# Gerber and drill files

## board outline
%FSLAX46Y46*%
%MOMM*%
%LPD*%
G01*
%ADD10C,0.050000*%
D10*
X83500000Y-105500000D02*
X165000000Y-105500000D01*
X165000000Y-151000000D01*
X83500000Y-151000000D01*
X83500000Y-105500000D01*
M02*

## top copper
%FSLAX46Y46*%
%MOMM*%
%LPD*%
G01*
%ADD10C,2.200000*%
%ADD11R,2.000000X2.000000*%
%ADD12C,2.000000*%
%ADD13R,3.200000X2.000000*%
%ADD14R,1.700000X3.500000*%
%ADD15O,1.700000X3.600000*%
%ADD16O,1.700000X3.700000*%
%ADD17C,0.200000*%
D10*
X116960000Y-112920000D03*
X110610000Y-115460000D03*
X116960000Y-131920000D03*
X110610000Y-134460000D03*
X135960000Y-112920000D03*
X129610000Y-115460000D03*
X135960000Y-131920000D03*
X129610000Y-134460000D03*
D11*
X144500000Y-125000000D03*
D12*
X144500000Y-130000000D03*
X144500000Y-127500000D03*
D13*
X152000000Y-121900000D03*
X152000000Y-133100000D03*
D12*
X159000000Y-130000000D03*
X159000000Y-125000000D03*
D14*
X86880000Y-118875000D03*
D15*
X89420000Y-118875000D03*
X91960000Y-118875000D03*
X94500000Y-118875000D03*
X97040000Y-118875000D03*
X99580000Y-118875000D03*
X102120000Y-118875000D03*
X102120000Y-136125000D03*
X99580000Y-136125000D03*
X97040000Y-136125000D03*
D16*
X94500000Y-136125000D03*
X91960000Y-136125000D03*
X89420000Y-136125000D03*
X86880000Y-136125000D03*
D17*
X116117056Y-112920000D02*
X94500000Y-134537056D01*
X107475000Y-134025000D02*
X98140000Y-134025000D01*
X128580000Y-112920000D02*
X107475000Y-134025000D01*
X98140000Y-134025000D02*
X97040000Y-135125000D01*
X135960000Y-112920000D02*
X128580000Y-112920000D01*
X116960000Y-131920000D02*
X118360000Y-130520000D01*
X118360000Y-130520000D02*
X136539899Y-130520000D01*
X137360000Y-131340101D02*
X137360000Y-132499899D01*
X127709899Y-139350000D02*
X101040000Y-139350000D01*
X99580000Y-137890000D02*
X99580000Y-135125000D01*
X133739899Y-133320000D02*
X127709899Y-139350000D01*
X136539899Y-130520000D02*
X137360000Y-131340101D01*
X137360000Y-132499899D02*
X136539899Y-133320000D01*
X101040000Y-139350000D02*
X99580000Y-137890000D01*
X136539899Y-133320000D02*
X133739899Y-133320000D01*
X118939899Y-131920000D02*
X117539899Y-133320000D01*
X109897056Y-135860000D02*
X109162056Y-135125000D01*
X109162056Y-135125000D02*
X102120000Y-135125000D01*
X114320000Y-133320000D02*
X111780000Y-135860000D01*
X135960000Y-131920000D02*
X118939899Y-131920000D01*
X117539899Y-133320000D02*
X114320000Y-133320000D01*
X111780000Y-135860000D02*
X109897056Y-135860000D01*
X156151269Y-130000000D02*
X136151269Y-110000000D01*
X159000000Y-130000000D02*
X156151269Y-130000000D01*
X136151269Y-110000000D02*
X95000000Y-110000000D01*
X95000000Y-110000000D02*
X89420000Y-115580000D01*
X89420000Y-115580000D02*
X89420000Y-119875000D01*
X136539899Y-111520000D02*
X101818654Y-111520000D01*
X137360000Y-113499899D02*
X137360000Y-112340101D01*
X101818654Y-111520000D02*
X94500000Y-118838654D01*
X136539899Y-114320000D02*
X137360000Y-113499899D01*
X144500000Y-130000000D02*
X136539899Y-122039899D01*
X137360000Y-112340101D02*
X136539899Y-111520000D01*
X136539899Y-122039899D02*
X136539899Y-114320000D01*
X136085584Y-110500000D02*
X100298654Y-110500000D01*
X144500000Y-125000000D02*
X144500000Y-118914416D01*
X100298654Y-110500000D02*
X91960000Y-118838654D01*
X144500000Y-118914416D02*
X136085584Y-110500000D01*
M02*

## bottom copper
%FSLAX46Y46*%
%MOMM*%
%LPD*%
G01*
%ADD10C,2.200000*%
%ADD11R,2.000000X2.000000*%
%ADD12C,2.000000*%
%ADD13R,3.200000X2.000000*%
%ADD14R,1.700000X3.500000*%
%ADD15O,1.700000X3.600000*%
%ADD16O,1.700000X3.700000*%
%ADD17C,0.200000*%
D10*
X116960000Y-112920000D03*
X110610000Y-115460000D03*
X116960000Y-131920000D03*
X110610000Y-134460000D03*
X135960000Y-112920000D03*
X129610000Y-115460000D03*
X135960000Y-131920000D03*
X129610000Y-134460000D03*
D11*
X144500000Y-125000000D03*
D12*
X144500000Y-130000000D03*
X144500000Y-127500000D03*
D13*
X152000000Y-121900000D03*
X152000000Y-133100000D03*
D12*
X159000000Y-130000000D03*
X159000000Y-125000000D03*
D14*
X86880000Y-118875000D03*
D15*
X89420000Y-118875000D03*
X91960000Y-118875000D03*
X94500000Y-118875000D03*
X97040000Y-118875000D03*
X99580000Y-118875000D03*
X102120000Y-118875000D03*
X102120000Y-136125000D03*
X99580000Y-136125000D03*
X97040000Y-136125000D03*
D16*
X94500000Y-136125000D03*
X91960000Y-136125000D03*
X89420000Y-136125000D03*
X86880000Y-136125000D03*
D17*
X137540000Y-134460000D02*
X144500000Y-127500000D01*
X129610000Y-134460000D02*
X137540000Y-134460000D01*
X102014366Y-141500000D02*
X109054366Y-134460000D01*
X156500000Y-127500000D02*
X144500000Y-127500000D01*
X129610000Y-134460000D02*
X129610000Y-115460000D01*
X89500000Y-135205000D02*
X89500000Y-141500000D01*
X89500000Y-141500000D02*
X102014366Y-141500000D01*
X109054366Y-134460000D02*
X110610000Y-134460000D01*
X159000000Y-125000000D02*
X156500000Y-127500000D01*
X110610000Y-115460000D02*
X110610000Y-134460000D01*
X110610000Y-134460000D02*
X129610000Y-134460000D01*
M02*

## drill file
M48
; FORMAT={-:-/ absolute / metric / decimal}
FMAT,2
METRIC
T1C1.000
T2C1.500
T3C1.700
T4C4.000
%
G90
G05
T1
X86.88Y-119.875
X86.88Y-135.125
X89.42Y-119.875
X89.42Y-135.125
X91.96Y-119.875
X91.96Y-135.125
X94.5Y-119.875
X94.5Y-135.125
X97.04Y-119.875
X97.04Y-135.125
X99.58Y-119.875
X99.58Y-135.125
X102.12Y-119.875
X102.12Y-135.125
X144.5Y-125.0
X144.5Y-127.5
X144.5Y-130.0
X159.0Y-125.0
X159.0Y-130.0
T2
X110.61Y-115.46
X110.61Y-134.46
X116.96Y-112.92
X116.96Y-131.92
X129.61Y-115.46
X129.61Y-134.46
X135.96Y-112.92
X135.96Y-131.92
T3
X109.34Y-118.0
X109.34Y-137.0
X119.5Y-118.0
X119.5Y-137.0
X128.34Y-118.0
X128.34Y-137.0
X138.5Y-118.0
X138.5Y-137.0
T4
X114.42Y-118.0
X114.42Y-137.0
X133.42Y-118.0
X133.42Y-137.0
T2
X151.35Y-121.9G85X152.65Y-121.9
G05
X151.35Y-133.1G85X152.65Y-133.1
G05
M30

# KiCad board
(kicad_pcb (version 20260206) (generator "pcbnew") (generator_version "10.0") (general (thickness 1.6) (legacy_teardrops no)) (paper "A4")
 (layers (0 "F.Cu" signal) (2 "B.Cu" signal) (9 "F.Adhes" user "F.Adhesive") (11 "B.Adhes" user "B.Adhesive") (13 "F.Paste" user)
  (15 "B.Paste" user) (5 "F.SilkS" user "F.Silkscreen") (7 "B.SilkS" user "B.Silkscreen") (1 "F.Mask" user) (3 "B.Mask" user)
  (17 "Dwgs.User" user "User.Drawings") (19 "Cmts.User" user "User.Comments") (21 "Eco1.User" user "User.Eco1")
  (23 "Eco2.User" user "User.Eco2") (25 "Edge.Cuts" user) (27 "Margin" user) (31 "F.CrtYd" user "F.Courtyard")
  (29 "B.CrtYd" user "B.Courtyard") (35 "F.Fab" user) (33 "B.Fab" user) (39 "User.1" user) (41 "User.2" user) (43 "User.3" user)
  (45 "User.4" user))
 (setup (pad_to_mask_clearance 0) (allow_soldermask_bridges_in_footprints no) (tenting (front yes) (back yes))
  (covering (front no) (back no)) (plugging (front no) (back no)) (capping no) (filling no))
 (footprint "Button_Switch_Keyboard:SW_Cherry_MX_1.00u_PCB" (layer "F.Cu") (at 116.96 112.92)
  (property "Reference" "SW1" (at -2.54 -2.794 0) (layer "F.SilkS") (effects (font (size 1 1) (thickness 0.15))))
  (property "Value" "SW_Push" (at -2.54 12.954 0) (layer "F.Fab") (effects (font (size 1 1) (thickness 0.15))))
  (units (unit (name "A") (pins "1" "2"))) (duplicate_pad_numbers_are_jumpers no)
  (pad "" np_thru_hole circle (at -7.62 5.08) (size 1.7 1.7) (drill 1.7) (layers "*.Cu" "*.Mask"))
  (pad "" np_thru_hole circle (at -2.54 5.08) (size 4 4) (drill 4) (layers "*.Cu" "*.Mask"))
  (pad "" np_thru_hole circle (at 2.54 5.08) (size 1.7 1.7) (drill 1.7) (layers "*.Cu" "*.Mask"))
  (pad "1" thru_hole circle (at 0 0) (size 2.2 2.2) (drill 1.5) (layers "*.Cu" "*.Mask") (remove_unused_layers no)
   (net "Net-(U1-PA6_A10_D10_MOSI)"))
  (pad "2" thru_hole circle (at -6.35 2.54) (size 2.2 2.2) (drill 1.5) (layers "*.Cu" "*.Mask") (remove_unused_layers no)
   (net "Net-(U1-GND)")))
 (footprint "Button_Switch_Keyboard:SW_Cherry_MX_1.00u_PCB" (layer "F.Cu") (at 116.96 131.92)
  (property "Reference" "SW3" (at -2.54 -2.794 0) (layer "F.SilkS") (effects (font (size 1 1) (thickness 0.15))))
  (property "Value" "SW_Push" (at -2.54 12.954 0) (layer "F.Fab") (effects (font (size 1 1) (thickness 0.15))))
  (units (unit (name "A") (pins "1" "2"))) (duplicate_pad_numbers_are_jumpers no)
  (pad "" np_thru_hole circle (at -7.62 5.08) (size 1.7 1.7) (drill 1.7) (layers "*.Cu" "*.Mask"))
  (pad "" np_thru_hole circle (at -2.54 5.08) (size 4 4) (drill 4) (layers "*.Cu" "*.Mask"))
  (pad "" np_thru_hole circle (at 2.54 5.08) (size 1.7 1.7) (drill 1.7) (layers "*.Cu" "*.Mask"))
  (pad "1" thru_hole circle (at 0 0) (size 2.2 2.2) (drill 1.5) (layers "*.Cu" "*.Mask") (remove_unused_layers no)
   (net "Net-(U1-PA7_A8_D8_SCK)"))
  (pad "2" thru_hole circle (at -6.35 2.54) (size 2.2 2.2) (drill 1.5) (layers "*.Cu" "*.Mask") (remove_unused_layers no)
   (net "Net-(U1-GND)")))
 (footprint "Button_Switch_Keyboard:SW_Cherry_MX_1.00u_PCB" (layer "F.Cu") (at 135.96 112.92)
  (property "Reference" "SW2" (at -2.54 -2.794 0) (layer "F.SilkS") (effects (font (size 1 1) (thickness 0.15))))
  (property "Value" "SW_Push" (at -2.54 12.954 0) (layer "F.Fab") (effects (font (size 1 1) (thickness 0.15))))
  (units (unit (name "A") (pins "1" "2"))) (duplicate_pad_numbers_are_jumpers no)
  (pad "" np_thru_hole circle (at -7.62 5.08) (size 1.7 1.7) (drill 1.7) (layers "*.Cu" "*.Mask"))
  (pad "" np_thru_hole circle (at -2.54 5.08) (size 4 4) (drill 4) (layers "*.Cu" "*.Mask"))
  (pad "" np_thru_hole circle (at 2.54 5.08) (size 1.7 1.7) (drill 1.7) (layers "*.Cu" "*.Mask"))
  (pad "1" thru_hole circle (at 0 0) (size 2.2 2.2) (drill 1.5) (layers "*.Cu" "*.Mask") (remove_unused_layers no)
   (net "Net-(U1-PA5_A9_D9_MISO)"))
  (pad "2" thru_hole circle (at -6.35 2.54) (size 2.2 2.2) (drill 1.5) (layers "*.Cu" "*.Mask") (remove_unused_layers no)
   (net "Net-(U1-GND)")))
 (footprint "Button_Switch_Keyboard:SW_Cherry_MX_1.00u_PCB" (layer "F.Cu") (at 135.96 131.92)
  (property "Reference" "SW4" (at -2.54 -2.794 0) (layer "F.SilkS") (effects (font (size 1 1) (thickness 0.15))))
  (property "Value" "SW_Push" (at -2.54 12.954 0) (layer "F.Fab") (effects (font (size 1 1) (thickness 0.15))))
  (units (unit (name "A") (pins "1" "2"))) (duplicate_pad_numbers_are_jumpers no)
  (pad "" np_thru_hole circle (at -7.62 5.08) (size 1.7 1.7) (drill 1.7) (layers "*.Cu" "*.Mask"))
  (pad "" np_thru_hole circle (at -2.54 5.08) (size 4 4) (drill 4) (layers "*.Cu" "*.Mask"))
  (pad "" np_thru_hole circle (at 2.54 5.08) (size 1.7 1.7) (drill 1.7) (layers "*.Cu" "*.Mask"))
  (pad "1" thru_hole circle (at 0 0) (size 2.2 2.2) (drill 1.5) (layers "*.Cu" "*.Mask") (remove_unused_layers no)
   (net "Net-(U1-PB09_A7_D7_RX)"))
  (pad "2" thru_hole circle (at -6.35 2.54) (size 2.2 2.2) (drill 1.5) (layers "*.Cu" "*.Mask") (remove_unused_layers no)
   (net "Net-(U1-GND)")))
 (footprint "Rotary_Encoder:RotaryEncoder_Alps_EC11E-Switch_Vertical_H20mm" (layer "F.Cu") (at 144.5 125)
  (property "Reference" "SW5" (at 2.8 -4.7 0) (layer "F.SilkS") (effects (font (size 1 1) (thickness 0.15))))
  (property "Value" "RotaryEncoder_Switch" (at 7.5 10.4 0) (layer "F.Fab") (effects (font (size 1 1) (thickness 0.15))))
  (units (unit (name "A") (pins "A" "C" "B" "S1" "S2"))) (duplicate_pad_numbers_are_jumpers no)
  (pad "A" thru_hole rect (at 0 0) (size 2 2) (drill 1) (layers "*.Cu" "*.Mask") (remove_unused_layers no) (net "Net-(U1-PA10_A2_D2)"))
  (pad "B" thru_hole circle (at 0 5) (size 2 2) (drill 1) (layers "*.Cu" "*.Mask") (remove_unused_layers no) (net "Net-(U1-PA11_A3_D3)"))
  (pad "C" thru_hole circle (at 0 2.5) (size 2 2) (drill 1) (layers "*.Cu" "*.Mask") (remove_unused_layers no) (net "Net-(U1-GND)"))
  (pad "MP" thru_hole rect (at 7.5 -3.1) (size 3.2 2) (drill oval 2.8 1.5) (layers "*.Cu" "*.Mask") (remove_unused_layers no))
  (pad "MP" thru_hole rect (at 7.5 8.1) (size 3.2 2) (drill oval 2.8 1.5) (layers "*.Cu" "*.Mask") (remove_unused_layers no))
  (pad "S1" thru_hole circle (at 14.5 5) (size 2 2) (drill 1) (layers "*.Cu" "*.Mask") (remove_unused_layers no) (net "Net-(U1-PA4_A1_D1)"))
  (pad "S2" thru_hole circle (at 14.5 0) (size 2 2) (drill 1) (layers "*.Cu" "*.Mask") (remove_unused_layers no) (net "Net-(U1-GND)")))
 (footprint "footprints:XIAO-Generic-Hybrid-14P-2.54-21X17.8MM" (layer "B.Cu") (at 94.5 127.5 -90)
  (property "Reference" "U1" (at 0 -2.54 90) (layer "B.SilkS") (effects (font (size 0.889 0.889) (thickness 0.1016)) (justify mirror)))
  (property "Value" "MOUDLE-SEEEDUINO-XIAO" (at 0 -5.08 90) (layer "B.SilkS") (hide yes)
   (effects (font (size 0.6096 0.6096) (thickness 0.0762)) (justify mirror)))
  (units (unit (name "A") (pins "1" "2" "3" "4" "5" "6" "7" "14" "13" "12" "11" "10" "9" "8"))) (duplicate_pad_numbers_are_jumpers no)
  (pad "1" thru_hole rect (at -7.625 7.62 270) (size 3.5 1.7) (drill 1 (offset -1 0)) (layers "*.Cu" "*.Mask") (remove_unused_layers no)
   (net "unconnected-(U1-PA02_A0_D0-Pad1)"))
  (pad "2" thru_hole oval (at -7.625 5.08 270) (size 3.6 1.7) (drill 1 (offset -1 0)) (layers "*.Cu" "*.Mask") (remove_unused_layers no)
   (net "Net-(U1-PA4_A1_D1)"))
  (pad "3" thru_hole oval (at -7.625 2.54 270) (size 3.6 1.7) (drill 1 (offset -1 0)) (layers "*.Cu" "*.Mask") (remove_unused_layers no)
   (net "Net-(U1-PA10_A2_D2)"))
  (pad "4" thru_hole oval (at -7.625 0 270) (size 3.6 1.7) (drill 1 (offset -1 0)) (layers "*.Cu" "*.Mask") (remove_unused_layers no)
   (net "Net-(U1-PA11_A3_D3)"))
  (pad "5" thru_hole oval (at -7.625 -2.54 270) (size 3.6 1.7) (drill 1 (offset -1 0)) (layers "*.Cu" "*.Mask") (remove_unused_layers no)
   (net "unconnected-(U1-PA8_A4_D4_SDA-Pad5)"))
  (pad "6" thru_hole oval (at -7.625 -5.08 90) (size 3.6 1.7) (drill 1 (offset 1 0)) (layers "*.Cu" "*.Mask") (remove_unused_layers no)
   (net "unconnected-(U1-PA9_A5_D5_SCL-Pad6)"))
  (pad "7" thru_hole oval (at -7.625 -7.62 270) (size 3.6 1.7) (drill 1 (offset -1 0)) (layers "*.Cu" "*.Mask") (remove_unused_layers no)
   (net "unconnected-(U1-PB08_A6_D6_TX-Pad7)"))
  (pad "8" thru_hole oval (at 7.625 -7.62 270) (size 3.6 1.7) (drill 1 (offset 1 0)) (layers "*.Cu" "*.Mask") (remove_unused_layers no)
   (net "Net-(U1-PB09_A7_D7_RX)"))
  (pad "9" thru_hole oval (at 7.625 -5.08 270) (size 3.6 1.7) (drill 1 (offset 1 0)) (layers "*.Cu" "*.Mask") (remove_unused_layers no)
   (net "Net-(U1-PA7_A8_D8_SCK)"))
  (pad "10" thru_hole oval (at 7.625 -2.54 270) (size 3.6 1.7) (drill 1 (offset 1 0)) (layers "*.Cu" "*.Mask") (remove_unused_layers no)
   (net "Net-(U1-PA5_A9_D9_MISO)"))
  (pad "11" thru_hole oval (at 7.625 0 270) (size 3.7 1.7) (drill 1 (offset 1 0)) (layers "*.Cu" "*.Mask") (remove_unused_layers no)
   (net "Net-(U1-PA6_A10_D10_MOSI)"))
  (pad "12" thru_hole oval (at 7.625 2.54 270) (size 3.7 1.7) (drill 1 (offset 1 0)) (layers "*.Cu" "*.Mask") (remove_unused_layers no)
   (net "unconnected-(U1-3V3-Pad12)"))
  (pad "13" thru_hole oval (at 7.625 5.08 270) (size 3.7 1.7) (drill 1 (offset 1 0)) (layers "*.Cu" "*.Mask") (remove_unused_layers no)
   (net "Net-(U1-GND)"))
  (pad "14" thru_hole oval (at 7.625 7.62 270) (size 3.7 1.7) (drill 1 (offset 1 0)) (layers "*.Cu" "*.Mask") (remove_unused_layers no)
   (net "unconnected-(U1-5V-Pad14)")))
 (gr_rect (start 83.5 105.5) (end 165 151) (stroke (width 0.05) (type default)) (fill no) (layer "Edge.Cuts"))
 (segment (start 116.117056 112.92) (end 94.5 134.537056) (width 0.2) (layer "F.Cu") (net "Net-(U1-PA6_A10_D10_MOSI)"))
 (segment (start 137.54 134.46) (end 144.5 127.5) (width 0.2) (layer "B.Cu") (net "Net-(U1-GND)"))
 (segment (start 129.61 134.46) (end 137.54 134.46) (width 0.2) (layer "B.Cu") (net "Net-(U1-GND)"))
 (segment (start 102.014366 141.5) (end 109.054366 134.46) (width 0.2) (layer "B.Cu") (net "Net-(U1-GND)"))
 (segment (start 156.5 127.5) (end 144.5 127.5) (width 0.2) (layer "B.Cu") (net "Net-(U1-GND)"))
 (segment (start 129.61 134.46) (end 129.61 115.46) (width 0.2) (layer "B.Cu") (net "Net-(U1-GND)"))
 (segment (start 89.5 135.205) (end 89.5 141.5) (width 0.2) (layer "B.Cu") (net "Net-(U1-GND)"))
 (segment (start 89.5 141.5) (end 102.014366 141.5) (width 0.2) (layer "B.Cu") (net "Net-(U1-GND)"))
 (segment (start 109.054366 134.46) (end 110.61 134.46) (width 0.2) (layer "B.Cu") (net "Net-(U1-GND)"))
 (segment (start 159 125) (end 156.5 127.5) (width 0.2) (layer "B.Cu") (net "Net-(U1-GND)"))
 (segment (start 110.61 115.46) (end 110.61 134.46) (width 0.2) (layer "B.Cu") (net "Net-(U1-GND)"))
 (segment (start 110.61 134.46) (end 129.61 134.46) (width 0.2) (layer "B.Cu") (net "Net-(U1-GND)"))
 (segment (start 107.475 134.025) (end 98.14 134.025) (width 0.2) (layer "F.Cu") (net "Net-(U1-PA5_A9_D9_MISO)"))
 (segment (start 128.58 112.92) (end 107.475 134.025) (width 0.2) (layer "F.Cu") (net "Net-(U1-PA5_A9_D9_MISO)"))
 (segment (start 98.14 134.025) (end 97.04 135.125) (width 0.2) (layer "F.Cu") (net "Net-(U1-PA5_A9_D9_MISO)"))
 (segment (start 135.96 112.92) (end 128.58 112.92) (width 0.2) (layer "F.Cu") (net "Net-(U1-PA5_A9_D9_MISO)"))
 (segment (start 116.96 131.92) (end 118.36 130.52) (width 0.2) (layer "F.Cu") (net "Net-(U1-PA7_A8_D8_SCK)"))
 (segment (start 118.36 130.52) (end 136.539899 130.52) (width 0.2) (layer "F.Cu") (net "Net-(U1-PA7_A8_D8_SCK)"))
 (segment (start 137.36 131.340101) (end 137.36 132.499899) (width 0.2) (layer "F.Cu") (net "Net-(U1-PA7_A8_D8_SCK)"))
 (segment (start 127.709899 139.35) (end 101.04 139.35) (width 0.2) (layer "F.Cu") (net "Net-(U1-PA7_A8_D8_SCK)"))
 (segment (start 99.58 137.89) (end 99.58 135.125) (width 0.2) (layer "F.Cu") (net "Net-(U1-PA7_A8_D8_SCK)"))
 (segment (start 133.739899 133.32) (end 127.709899 139.35) (width 0.2) (layer "F.Cu") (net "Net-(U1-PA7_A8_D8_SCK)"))
 (segment (start 136.539899 130.52) (end 137.36 131.340101) (width 0.2) (layer "F.Cu") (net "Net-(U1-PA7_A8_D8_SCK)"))
 (segment (start 137.36 132.499899) (end 136.539899 133.32) (width 0.2) (layer "F.Cu") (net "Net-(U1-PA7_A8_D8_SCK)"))
 (segment (start 101.04 139.35) (end 99.58 137.89) (width 0.2) (layer "F.Cu") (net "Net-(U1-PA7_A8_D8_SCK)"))
 (segment (start 136.539899 133.32) (end 133.739899 133.32) (width 0.2) (layer "F.Cu") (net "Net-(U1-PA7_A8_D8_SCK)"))
 (segment (start 118.939899 131.92) (end 117.539899 133.32) (width 0.2) (layer "F.Cu") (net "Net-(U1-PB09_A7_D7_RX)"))
 (segment (start 109.897056 135.86) (end 109.162056 135.125) (width 0.2) (layer "F.Cu") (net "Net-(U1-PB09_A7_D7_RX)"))
 (segment (start 109.162056 135.125) (end 102.12 135.125) (width 0.2) (layer "F.Cu") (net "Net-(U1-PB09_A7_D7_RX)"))
 (segment (start 114.32 133.32) (end 111.78 135.86) (width 0.2) (layer "F.Cu") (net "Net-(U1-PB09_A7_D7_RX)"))
 (segment (start 135.96 131.92) (end 118.939899 131.92) (width 0.2) (layer "F.Cu") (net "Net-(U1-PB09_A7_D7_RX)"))
 (segment (start 117.539899 133.32) (end 114.32 133.32) (width 0.2) (layer "F.Cu") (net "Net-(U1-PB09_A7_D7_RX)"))
 (segment (start 111.78 135.86) (end 109.897056 135.86) (width 0.2) (layer "F.Cu") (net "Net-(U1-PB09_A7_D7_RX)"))
 (segment (start 156.151269 130) (end 136.151269 110) (width 0.2) (layer "F.Cu") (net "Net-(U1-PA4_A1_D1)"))
 (segment (start 159 130) (end 156.151269 130) (width 0.2) (layer "F.Cu") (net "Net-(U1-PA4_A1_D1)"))
 (segment (start 136.151269 110) (end 95 110) (width 0.2) (layer "F.Cu") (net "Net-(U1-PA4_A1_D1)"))
 (segment (start 95 110) (end 89.42 115.58) (width 0.2) (layer "F.Cu") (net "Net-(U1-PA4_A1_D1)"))
 (segment (start 89.42 115.58) (end 89.42 119.875) (width 0.2) (layer "F.Cu") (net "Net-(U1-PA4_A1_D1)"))
 (segment (start 136.539899 111.52) (end 101.818654 111.52) (width 0.2) (layer "F.Cu") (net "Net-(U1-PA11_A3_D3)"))
 (segment (start 137.36 113.499899) (end 137.36 112.340101) (width 0.2) (layer "F.Cu") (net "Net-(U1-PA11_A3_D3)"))
 (segment (start 101.818654 111.52) (end 94.5 118.838654) (width 0.2) (layer "F.Cu") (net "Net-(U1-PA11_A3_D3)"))
 (segment (start 136.539899 114.32) (end 137.36 113.499899) (width 0.2) (layer "F.Cu") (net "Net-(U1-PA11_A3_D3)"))
 (segment (start 144.5 130) (end 136.539899 122.039899) (width 0.2) (layer "F.Cu") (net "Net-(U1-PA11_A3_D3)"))
 (segment (start 137.36 112.340101) (end 136.539899 111.52) (width 0.2) (layer "F.Cu") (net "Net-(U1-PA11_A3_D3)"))
 (segment (start 136.539899 122.039899) (end 136.539899 114.32) (width 0.2) (layer "F.Cu") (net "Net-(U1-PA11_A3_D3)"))
 (segment (start 136.085584 110.5) (end 100.298654 110.5) (width 0.2) (layer "F.Cu") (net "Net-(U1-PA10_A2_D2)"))
 (segment (start 144.5 125) (end 144.5 118.914416) (width 0.2) (layer "F.Cu") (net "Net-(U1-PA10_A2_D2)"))
 (segment (start 100.298654 110.5) (end 91.96 118.838654) (width 0.2) (layer "F.Cu") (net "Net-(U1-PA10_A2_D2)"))
 (segment (start 144.5 118.914416) (end 136.085584 110.5) (width 0.2) (layer "F.Cu") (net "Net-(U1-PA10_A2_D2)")))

